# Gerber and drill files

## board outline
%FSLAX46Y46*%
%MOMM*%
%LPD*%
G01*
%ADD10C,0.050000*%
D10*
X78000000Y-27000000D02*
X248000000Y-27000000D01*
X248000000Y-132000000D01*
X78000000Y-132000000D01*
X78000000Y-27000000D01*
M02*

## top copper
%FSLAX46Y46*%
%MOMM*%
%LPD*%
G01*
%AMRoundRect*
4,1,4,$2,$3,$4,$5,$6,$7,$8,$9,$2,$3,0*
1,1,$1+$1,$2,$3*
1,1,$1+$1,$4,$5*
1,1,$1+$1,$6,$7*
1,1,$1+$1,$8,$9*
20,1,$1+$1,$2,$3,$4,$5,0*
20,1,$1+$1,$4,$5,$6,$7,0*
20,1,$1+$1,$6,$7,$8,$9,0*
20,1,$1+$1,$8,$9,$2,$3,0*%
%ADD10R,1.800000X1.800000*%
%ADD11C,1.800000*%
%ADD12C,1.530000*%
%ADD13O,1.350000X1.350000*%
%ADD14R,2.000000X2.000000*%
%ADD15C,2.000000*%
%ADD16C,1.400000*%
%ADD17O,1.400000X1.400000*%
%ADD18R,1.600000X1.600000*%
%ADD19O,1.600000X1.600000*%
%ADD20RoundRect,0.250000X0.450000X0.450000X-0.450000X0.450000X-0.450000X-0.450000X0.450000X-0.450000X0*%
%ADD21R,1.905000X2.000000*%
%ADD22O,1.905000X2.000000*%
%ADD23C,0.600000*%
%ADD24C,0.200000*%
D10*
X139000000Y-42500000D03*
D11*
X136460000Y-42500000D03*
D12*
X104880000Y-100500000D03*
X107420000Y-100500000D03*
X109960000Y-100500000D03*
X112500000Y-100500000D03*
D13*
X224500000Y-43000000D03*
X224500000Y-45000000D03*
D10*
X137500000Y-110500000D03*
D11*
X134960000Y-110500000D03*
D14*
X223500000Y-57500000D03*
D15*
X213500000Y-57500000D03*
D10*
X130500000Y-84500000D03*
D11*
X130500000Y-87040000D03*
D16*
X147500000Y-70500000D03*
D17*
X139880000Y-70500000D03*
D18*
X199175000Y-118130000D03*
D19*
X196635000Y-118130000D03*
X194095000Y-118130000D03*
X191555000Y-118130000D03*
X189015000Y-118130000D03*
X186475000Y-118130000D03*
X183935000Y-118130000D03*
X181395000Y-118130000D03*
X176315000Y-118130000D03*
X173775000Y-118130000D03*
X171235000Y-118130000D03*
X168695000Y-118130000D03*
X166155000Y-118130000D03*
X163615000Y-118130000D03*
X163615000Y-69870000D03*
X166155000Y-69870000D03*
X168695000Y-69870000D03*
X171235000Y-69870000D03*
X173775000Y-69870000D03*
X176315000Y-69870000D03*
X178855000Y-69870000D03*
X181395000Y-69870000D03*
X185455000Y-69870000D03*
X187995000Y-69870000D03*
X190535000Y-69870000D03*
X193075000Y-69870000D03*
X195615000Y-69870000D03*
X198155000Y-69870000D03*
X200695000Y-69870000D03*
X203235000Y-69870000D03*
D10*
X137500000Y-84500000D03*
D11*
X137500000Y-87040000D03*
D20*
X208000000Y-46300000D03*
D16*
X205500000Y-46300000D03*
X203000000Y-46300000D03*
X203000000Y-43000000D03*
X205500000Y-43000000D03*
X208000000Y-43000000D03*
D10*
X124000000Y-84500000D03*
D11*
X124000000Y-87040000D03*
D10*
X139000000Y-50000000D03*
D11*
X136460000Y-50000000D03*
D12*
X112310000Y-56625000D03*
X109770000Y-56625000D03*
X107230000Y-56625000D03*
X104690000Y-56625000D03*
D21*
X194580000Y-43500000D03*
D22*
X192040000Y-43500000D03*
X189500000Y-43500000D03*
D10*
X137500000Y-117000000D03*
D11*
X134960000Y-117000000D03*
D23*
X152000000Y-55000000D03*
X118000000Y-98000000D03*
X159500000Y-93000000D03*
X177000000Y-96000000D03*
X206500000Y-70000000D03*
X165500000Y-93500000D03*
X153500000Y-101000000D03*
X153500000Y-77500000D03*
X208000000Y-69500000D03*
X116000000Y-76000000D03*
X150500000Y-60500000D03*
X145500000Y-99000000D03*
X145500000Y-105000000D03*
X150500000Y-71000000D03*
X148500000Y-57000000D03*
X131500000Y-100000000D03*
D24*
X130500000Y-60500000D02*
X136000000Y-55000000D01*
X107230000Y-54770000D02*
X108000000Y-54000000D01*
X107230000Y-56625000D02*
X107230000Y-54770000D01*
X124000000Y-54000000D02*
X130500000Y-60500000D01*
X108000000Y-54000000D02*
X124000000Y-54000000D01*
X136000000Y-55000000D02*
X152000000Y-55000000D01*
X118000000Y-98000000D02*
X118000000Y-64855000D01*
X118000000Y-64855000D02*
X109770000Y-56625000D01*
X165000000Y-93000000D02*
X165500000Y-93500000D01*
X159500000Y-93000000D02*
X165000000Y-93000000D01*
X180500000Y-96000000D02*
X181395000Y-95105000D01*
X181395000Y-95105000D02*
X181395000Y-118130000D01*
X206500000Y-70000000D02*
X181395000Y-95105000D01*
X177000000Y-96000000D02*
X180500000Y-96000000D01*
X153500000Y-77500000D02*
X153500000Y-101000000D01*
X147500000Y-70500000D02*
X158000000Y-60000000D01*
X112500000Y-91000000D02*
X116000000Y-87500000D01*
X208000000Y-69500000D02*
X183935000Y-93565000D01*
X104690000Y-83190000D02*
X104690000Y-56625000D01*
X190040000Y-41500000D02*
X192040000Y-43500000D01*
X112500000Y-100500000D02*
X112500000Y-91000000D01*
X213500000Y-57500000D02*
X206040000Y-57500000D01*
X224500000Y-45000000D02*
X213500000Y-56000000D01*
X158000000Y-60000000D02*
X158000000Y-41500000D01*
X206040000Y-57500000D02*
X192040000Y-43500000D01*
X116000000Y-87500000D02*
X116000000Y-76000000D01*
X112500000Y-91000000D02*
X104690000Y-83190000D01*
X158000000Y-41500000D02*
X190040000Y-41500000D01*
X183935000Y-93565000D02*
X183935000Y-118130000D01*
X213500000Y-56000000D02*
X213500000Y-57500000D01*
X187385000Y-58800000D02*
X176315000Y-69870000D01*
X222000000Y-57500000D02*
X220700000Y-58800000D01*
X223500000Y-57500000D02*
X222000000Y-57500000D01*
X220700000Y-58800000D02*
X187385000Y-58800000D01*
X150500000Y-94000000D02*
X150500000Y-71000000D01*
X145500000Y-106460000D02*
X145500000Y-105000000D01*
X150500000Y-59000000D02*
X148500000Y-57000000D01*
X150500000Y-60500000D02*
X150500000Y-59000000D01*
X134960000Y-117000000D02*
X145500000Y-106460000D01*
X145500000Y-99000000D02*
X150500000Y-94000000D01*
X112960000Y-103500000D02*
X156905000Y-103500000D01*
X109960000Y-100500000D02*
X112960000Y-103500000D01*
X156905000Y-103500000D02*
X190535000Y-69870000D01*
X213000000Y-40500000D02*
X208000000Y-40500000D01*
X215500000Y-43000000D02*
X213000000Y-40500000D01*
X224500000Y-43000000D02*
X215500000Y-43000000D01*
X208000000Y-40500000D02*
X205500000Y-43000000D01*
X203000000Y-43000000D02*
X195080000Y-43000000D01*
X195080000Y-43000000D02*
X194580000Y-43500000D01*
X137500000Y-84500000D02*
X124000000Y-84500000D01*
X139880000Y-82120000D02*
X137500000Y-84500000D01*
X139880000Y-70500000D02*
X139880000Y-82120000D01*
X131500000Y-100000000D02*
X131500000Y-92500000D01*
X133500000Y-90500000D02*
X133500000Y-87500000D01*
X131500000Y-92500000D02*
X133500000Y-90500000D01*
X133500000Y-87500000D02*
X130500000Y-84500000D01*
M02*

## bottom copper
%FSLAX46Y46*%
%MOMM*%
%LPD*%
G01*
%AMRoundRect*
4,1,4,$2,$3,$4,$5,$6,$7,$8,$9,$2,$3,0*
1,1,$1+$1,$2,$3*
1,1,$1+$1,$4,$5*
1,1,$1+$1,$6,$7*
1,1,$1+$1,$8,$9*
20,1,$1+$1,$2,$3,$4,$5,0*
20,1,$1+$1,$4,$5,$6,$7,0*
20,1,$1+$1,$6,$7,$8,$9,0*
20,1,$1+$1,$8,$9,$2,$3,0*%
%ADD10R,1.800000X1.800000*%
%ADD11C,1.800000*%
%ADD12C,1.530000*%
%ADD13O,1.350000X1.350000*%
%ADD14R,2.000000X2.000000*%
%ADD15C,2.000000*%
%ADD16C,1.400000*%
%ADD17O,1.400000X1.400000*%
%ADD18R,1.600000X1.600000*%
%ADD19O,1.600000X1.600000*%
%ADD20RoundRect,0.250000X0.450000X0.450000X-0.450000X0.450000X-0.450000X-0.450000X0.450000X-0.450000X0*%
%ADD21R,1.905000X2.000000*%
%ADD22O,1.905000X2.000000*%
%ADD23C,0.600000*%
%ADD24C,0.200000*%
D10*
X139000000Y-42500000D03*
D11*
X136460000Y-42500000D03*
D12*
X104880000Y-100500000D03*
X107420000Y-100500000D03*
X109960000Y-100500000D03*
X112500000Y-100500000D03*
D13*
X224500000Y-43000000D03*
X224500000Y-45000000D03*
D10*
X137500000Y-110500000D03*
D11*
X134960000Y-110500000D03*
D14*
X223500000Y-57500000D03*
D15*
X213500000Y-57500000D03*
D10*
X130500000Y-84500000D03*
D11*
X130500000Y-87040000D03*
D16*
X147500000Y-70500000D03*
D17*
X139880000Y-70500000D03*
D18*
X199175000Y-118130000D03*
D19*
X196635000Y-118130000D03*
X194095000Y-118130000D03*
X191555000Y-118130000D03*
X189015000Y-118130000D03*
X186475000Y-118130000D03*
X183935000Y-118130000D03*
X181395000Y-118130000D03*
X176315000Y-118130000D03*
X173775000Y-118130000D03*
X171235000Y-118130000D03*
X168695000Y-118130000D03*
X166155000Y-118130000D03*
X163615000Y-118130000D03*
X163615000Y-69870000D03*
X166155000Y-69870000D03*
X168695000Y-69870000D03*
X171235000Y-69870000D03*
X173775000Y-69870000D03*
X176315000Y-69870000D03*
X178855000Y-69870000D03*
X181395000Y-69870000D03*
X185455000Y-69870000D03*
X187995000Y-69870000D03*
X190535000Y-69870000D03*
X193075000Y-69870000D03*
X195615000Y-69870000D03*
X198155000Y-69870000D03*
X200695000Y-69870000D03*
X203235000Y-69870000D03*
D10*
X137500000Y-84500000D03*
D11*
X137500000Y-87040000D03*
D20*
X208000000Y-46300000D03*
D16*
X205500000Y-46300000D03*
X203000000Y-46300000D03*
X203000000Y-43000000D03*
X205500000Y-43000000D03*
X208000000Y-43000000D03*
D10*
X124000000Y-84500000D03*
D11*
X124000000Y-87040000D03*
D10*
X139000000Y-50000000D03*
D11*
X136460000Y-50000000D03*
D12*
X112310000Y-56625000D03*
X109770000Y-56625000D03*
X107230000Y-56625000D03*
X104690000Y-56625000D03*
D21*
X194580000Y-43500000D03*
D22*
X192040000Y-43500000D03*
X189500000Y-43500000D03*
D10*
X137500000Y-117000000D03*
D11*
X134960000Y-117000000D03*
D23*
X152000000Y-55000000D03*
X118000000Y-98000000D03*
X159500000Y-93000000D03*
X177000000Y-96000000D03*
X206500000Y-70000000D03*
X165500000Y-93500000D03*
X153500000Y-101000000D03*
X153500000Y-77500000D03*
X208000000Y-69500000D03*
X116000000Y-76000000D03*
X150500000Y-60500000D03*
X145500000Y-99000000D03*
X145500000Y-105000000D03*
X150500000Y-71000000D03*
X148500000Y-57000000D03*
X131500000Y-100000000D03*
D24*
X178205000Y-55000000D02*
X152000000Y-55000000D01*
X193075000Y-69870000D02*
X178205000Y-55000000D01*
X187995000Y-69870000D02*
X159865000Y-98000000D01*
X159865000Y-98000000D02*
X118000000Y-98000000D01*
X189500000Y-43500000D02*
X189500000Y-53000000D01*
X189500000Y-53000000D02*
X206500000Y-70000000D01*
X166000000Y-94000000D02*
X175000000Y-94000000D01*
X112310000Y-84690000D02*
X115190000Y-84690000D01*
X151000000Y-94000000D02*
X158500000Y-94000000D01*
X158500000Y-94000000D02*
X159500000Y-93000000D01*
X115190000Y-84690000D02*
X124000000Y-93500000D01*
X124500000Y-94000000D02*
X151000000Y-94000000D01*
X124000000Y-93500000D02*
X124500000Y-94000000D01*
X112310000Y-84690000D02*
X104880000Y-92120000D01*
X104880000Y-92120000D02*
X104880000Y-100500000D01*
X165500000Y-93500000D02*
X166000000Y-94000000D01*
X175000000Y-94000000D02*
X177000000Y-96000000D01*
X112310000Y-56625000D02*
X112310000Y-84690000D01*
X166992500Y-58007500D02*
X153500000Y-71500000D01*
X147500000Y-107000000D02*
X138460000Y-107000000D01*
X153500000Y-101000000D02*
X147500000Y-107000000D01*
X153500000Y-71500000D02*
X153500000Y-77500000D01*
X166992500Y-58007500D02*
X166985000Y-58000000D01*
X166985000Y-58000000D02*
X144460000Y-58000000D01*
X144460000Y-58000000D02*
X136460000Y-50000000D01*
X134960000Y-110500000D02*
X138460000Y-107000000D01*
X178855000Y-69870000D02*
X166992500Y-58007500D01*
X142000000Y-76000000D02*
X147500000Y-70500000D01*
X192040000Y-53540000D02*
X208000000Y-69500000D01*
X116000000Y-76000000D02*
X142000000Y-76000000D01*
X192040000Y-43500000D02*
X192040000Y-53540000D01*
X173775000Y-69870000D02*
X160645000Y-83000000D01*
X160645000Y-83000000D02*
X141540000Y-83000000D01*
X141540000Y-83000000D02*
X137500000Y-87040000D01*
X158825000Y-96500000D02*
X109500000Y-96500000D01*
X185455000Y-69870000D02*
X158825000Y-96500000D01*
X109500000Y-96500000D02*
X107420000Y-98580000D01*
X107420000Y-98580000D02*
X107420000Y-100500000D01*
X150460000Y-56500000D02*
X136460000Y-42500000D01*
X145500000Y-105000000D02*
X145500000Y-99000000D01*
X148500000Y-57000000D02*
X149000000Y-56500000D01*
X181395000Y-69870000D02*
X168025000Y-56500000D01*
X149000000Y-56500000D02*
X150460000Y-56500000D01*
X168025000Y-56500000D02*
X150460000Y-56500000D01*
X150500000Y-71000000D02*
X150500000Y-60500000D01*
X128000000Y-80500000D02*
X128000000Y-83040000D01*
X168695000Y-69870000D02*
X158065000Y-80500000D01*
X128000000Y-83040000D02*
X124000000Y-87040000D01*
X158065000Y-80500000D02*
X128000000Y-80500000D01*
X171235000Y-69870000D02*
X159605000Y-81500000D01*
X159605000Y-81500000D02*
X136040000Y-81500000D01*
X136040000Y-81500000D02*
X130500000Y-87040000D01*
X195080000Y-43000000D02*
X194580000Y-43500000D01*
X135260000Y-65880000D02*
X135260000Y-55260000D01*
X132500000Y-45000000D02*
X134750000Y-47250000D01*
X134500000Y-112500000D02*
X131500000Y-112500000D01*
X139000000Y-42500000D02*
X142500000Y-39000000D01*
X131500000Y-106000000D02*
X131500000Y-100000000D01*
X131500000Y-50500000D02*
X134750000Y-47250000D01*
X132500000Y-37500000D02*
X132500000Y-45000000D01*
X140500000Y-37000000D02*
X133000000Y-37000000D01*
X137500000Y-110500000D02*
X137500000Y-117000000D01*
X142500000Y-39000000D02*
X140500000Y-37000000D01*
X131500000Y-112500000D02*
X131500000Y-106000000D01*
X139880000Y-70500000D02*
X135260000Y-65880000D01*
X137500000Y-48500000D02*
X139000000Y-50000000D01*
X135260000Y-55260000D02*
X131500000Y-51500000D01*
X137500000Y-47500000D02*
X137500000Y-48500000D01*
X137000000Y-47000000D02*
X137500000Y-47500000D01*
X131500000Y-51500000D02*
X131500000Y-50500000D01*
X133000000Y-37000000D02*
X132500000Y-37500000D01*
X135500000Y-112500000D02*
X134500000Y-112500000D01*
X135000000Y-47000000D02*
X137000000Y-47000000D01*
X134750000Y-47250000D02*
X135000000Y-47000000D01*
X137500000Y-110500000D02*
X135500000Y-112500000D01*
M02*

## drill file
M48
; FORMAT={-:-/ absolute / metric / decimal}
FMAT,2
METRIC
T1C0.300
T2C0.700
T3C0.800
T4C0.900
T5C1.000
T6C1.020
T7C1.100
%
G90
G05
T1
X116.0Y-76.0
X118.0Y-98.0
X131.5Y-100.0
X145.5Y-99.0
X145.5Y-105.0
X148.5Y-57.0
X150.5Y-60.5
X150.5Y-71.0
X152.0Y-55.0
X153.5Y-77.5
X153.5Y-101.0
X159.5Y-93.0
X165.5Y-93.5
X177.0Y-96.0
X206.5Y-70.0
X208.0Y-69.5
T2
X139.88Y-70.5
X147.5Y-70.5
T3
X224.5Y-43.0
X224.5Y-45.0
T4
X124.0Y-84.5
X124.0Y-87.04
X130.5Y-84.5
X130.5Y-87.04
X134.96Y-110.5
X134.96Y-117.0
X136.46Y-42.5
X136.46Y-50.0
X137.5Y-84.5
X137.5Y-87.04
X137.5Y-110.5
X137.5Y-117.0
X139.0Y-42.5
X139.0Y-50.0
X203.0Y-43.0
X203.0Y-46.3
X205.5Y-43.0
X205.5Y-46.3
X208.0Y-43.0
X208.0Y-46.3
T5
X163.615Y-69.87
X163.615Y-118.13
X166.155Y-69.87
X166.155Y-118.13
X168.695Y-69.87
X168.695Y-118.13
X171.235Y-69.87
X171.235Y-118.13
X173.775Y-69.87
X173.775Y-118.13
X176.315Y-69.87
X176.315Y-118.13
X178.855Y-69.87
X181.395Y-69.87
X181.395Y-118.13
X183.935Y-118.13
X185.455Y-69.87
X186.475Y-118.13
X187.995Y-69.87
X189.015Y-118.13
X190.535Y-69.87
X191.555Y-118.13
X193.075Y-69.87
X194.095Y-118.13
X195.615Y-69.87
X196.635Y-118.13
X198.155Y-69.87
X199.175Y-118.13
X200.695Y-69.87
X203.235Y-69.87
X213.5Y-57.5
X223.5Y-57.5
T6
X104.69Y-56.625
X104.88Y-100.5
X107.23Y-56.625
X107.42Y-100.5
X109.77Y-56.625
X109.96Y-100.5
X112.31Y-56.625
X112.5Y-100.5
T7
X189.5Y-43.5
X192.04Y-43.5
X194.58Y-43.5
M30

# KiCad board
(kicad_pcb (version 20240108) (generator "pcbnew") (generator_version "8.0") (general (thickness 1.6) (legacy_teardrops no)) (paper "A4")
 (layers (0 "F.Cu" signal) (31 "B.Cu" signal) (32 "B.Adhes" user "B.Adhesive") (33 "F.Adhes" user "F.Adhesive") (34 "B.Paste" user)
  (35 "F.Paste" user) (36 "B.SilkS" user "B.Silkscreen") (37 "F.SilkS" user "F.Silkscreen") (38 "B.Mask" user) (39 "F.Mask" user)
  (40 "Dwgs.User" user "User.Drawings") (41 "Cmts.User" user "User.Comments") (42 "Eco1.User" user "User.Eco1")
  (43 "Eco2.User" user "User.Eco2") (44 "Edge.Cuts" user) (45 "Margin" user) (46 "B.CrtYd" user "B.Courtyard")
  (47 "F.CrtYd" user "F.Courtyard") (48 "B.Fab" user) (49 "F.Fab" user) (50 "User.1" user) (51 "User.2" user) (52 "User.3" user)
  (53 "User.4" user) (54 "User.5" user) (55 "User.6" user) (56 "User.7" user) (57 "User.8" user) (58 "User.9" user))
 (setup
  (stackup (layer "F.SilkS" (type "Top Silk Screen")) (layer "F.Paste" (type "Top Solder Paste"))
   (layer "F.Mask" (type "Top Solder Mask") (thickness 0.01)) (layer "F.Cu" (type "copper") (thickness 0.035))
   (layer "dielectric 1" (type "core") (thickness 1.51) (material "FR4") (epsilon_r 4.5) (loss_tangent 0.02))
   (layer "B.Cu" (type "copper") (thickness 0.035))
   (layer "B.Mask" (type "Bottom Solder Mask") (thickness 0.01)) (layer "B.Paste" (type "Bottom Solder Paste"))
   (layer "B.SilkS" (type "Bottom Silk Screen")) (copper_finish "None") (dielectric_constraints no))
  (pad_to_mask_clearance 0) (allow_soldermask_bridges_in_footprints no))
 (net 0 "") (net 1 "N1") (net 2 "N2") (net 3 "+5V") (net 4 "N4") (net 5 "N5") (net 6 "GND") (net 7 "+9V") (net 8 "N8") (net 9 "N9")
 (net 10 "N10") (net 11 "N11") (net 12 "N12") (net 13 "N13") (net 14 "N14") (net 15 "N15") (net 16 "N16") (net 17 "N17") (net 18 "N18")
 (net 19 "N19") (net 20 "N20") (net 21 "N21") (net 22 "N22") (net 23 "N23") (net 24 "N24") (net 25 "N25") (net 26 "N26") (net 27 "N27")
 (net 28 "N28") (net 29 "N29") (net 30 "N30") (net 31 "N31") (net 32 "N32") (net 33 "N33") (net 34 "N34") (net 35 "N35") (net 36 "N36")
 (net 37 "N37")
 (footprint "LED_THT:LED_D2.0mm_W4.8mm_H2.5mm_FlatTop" (layer "F.Cu") (at 139 42.5 180)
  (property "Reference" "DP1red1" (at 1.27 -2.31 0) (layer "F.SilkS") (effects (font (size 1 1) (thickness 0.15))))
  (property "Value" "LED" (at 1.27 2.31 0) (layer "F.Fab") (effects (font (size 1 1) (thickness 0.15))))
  (pad "1" thru_hole rect (at 0 0 180) (size 1.8 1.8) (drill 0.9) (layers "*.Cu" "*.Mask") (remove_unused_layers no) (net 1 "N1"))
  (pad "2" thru_hole circle (at 2.54 0 180) (size 1.8 1.8) (drill 0.9) (layers "*.Cu" "*.Mask") (remove_unused_layers no) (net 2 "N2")))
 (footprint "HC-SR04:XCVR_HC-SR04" (layer "F.Cu") (at 108.69 100.5)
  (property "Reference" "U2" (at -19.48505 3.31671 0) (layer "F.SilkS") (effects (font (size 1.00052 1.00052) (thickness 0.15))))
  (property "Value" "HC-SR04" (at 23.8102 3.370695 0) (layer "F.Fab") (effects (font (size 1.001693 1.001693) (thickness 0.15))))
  (pad "1" thru_hole circle (at -3.81 0) (size 1.53 1.53) (drill 1.02) (layers "*.Cu" "*.Mask") (remove_unused_layers no) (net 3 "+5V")
   (solder_mask_margin 0.102))
  (pad "2" thru_hole circle (at -1.27 0) (size 1.53 1.53) (drill 1.02) (layers "*.Cu" "*.Mask") (remove_unused_layers no) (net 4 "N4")
   (solder_mask_margin 0.102))
  (pad "3" thru_hole circle (at 1.27 0) (size 1.53 1.53) (drill 1.02) (layers "*.Cu" "*.Mask") (remove_unused_layers no) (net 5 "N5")
   (solder_mask_margin 0.102))
  (pad "4" thru_hole circle (at 3.81 0) (size 1.53 1.53) (drill 1.02) (layers "*.Cu" "*.Mask") (remove_unused_layers no) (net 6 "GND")
   (solder_mask_margin 0.102)))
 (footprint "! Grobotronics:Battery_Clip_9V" (layer "F.Cu") (at 224.5 43.5)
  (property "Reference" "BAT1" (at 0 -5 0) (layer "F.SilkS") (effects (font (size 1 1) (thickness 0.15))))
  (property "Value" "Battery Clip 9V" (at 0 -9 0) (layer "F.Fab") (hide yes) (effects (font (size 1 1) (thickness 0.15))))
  (pad "+" thru_hole oval (at 0 -0.5) (size 1.35 1.35) (drill 0.8) (layers "*.Cu" "*.Mask") (remove_unused_layers no) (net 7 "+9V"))
  (pad "-" thru_hole oval (at 0 1.5) (size 1.35 1.35) (drill 0.8) (layers "*.Cu" "*.Mask") (remove_unused_layers no) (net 6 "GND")))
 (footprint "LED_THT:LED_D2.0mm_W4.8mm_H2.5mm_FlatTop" (layer "F.Cu") (at 137.5 110.5 180)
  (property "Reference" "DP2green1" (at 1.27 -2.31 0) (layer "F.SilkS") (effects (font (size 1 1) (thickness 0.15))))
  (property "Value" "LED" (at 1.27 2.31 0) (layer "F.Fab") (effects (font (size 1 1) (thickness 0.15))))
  (pad "1" thru_hole rect (at 0 0 180) (size 1.8 1.8) (drill 0.9) (layers "*.Cu" "*.Mask") (remove_unused_layers no) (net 1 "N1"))
  (pad "2" thru_hole circle (at 2.54 0 180) (size 1.8 1.8) (drill 0.9) (layers "*.Cu" "*.Mask") (remove_unused_layers no) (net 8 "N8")))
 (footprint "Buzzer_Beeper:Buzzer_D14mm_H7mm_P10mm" (layer "F.Cu") (at 223.5 57.5 180)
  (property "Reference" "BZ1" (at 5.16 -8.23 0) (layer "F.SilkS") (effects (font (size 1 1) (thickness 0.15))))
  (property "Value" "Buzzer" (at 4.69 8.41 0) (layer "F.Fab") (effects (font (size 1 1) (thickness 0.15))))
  (pad "1" thru_hole rect (at 0 0 180) (size 2 2) (drill 1) (layers "*.Cu" "*.Mask") (remove_unused_layers no) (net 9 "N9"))
  (pad "2" thru_hole circle (at 10 0 180) (size 2 2) (drill 1) (layers "*.Cu" "*.Mask") (remove_unused_layers no) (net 6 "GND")))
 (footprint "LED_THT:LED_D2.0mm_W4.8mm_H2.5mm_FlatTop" (layer "F.Cu") (at 130.5 84.5 -90)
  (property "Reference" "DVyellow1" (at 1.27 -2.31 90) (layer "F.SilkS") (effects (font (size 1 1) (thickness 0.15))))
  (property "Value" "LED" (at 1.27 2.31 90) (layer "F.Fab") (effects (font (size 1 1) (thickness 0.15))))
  (pad "1" thru_hole rect (at 0 0 270) (size 1.8 1.8) (drill 0.9) (layers "*.Cu" "*.Mask") (remove_unused_layers no) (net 1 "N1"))
  (pad "2" thru_hole circle (at 2.54 0 270) (size 1.8 1.8) (drill 0.9) (layers "*.Cu" "*.Mask") (remove_unused_layers no) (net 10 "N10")))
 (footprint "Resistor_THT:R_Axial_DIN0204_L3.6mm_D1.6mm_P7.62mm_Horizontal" (layer "F.Cu") (at 147.5 70.5 180)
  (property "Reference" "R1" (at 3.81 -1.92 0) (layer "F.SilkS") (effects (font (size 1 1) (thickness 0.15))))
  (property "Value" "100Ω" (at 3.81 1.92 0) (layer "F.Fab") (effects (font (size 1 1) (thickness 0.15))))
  (pad "1" thru_hole circle (at 0 0 180) (size 1.4 1.4) (drill 0.7) (layers "*.Cu" "*.Mask") (remove_unused_layers no) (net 6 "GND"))
  (pad "2" thru_hole oval (at 7.62 0 180) (size 1.4 1.4) (drill 0.7) (layers "*.Cu" "*.Mask") (remove_unused_layers no) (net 1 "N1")))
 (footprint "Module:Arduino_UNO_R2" (layer "F.Cu") (at 199.175 118.13 180)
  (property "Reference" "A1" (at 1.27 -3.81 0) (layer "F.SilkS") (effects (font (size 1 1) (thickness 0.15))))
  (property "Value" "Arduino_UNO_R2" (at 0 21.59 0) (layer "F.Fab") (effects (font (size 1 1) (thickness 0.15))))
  (pad "1" thru_hole rect (at 0 0 270) (size 1.6 1.6) (drill 1) (layers "*.Cu" "*.Mask") (remove_unused_layers no) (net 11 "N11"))
  (pad "2" thru_hole oval (at 2.54 0 270) (size 1.6 1.6) (drill 1) (layers "*.Cu" "*.Mask") (remove_unused_layers no) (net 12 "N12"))
  (pad "3" thru_hole oval (at 5.08 0 270) (size 1.6 1.6) (drill 1) (layers "*.Cu" "*.Mask") (remove_unused_layers no) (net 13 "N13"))
  (pad "4" thru_hole oval (at 7.62 0 270) (size 1.6 1.6) (drill 1) (layers "*.Cu" "*.Mask") (remove_unused_layers no) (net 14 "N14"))
  (pad "5" thru_hole oval (at 10.16 0 270) (size 1.6 1.6) (drill 1) (layers "*.Cu" "*.Mask") (remove_unused_layers no) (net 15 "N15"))
  (pad "6" thru_hole oval (at 12.7 0 270) (size 1.6 1.6) (drill 1) (layers "*.Cu" "*.Mask") (remove_unused_layers no) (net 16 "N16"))
  (pad "7" thru_hole oval (at 15.24 0 270) (size 1.6 1.6) (drill 1) (layers "*.Cu" "*.Mask") (remove_unused_layers no) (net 6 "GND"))
  (pad "8" thru_hole oval (at 17.78 0 270) (size 1.6 1.6) (drill 1) (layers "*.Cu" "*.Mask") (remove_unused_layers no) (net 3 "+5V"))
  (pad "9" thru_hole oval (at 22.86 0 270) (size 1.6 1.6) (drill 1) (layers "*.Cu" "*.Mask") (remove_unused_layers no) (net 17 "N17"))
  (pad "10" thru_hole oval (at 25.4 0 270) (size 1.6 1.6) (drill 1) (layers "*.Cu" "*.Mask") (remove_unused_layers no) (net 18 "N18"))
  (pad "11" thru_hole oval (at 27.94 0 270) (size 1.6 1.6) (drill 1) (layers "*.Cu" "*.Mask") (remove_unused_layers no) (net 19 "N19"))
  (pad "12" thru_hole oval (at 30.48 0 270) (size 1.6 1.6) (drill 1) (layers "*.Cu" "*.Mask") (remove_unused_layers no) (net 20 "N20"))
  (pad "13" thru_hole oval (at 33.02 0 270) (size 1.6 1.6) (drill 1) (layers "*.Cu" "*.Mask") (remove_unused_layers no) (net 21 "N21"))
  (pad "14" thru_hole oval (at 35.56 0 270) (size 1.6 1.6) (drill 1) (layers "*.Cu" "*.Mask") (remove_unused_layers no) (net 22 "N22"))
  (pad "15" thru_hole oval (at 35.56 48.26 270) (size 1.6 1.6) (drill 1) (layers "*.Cu" "*.Mask") (remove_unused_layers no) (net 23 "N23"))
  (pad "16" thru_hole oval (at 33.02 48.26 270) (size 1.6 1.6) (drill 1) (layers "*.Cu" "*.Mask") (remove_unused_layers no) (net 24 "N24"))
  (pad "17" thru_hole oval (at 30.48 48.26 270) (size 1.6 1.6) (drill 1) (layers "*.Cu" "*.Mask") (remove_unused_layers no) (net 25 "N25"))
  (pad "18" thru_hole oval (at 27.94 48.26 270) (size 1.6 1.6) (drill 1) (layers "*.Cu" "*.Mask") (remove_unused_layers no) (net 10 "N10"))
  (pad "19" thru_hole oval (at 25.4 48.26 270) (size 1.6 1.6) (drill 1) (layers "*.Cu" "*.Mask") (remove_unused_layers no) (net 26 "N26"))
  (pad "20" thru_hole oval (at 22.86 48.26 270) (size 1.6 1.6) (drill 1) (layers "*.Cu" "*.Mask") (remove_unused_layers no) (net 9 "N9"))
  (pad "21" thru_hole oval (at 20.32 48.26 270) (size 1.6 1.6) (drill 1) (layers "*.Cu" "*.Mask") (remove_unused_layers no) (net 8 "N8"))
  (pad "22" thru_hole oval (at 17.78 48.26 270) (size 1.6 1.6) (drill 1) (layers "*.Cu" "*.Mask") (remove_unused_layers no) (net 2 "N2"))
  (pad "23" thru_hole oval (at 13.72 48.26 270) (size 1.6 1.6) (drill 1) (layers "*.Cu" "*.Mask") (remove_unused_layers no) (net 4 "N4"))
  (pad "24" thru_hole oval (at 11.18 48.26 270) (size 1.6 1.6) (drill 1) (layers "*.Cu" "*.Mask") (remove_unused_layers no) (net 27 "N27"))
  (pad "25" thru_hole oval (at 8.64 48.26 270) (size 1.6 1.6) (drill 1) (layers "*.Cu" "*.Mask") (remove_unused_layers no) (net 5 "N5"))
  (pad "26" thru_hole oval (at 6.1 48.26 270) (size 1.6 1.6) (drill 1) (layers "*.Cu" "*.Mask") (remove_unused_layers no) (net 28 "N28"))
  (pad "27" thru_hole oval (at 3.56 48.26 270) (size 1.6 1.6) (drill 1) (layers "*.Cu" "*.Mask") (remove_unused_layers no) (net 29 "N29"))
  (pad "28" thru_hole oval (at 1.02 48.26 270) (size 1.6 1.6) (drill 1) (layers "*.Cu" "*.Mask") (remove_unused_layers no) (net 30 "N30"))
  (pad "29" thru_hole oval (at -1.52 48.26 270) (size 1.6 1.6) (drill 1) (layers "*.Cu" "*.Mask") (remove_unused_layers no) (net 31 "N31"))
  (pad "30" thru_hole oval (at -4.06 48.26 270) (size 1.6 1.6) (drill 1) (layers "*.Cu" "*.Mask") (remove_unused_layers no) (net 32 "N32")))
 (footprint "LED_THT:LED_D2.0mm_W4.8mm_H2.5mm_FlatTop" (layer "F.Cu") (at 137.5 84.5 -90)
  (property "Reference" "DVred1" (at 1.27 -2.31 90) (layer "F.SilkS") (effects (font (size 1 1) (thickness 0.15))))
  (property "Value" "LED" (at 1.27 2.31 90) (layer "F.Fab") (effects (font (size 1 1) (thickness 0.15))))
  (pad "1" thru_hole rect (at 0 0 270) (size 1.8 1.8) (drill 0.9) (layers "*.Cu" "*.Mask") (remove_unused_layers no) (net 1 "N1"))
  (pad "2" thru_hole circle (at 2.54 0 270) (size 1.8 1.8) (drill 0.9) (layers "*.Cu" "*.Mask") (remove_unused_layers no) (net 26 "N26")))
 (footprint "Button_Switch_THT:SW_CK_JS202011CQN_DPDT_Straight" (layer "F.Cu") (at 208 46.3 180)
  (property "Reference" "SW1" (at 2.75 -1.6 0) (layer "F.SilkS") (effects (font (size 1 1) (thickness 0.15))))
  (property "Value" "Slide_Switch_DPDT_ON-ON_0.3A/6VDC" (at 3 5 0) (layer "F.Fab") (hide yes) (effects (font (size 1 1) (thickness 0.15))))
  (pad "1" thru_hole roundrect (at 0 0 180) (size 1.4 1.4) (drill 0.9) (layers "*.Cu" "*.Mask") (remove_unused_layers no)
   (roundrect_rratio 0.1785714286) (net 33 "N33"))
  (pad "2" thru_hole circle (at 2.5 0 180) (size 1.4 1.4) (drill 0.9) (layers "*.Cu" "*.Mask") (remove_unused_layers no) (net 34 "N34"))
  (pad "3" thru_hole circle (at 5 0 180) (size 1.4 1.4) (drill 0.9) (layers "*.Cu" "*.Mask") (remove_unused_layers no) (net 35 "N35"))
  (pad "4" thru_hole circle (at 5 3.3 180) (size 1.4 1.4) (drill 0.9) (layers "*.Cu" "*.Mask") (remove_unused_layers no) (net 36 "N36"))
  (pad "5" thru_hole circle (at 2.5 3.3 180) (size 1.4 1.4) (drill 0.9) (layers "*.Cu" "*.Mask") (remove_unused_layers no) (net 7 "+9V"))
  (pad "6" thru_hole circle (at 0 3.3 180) (size 1.4 1.4) (drill 0.9) (layers "*.Cu" "*.Mask") (remove_unused_layers no) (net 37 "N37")))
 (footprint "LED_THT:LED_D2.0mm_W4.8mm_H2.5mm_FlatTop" (layer "F.Cu") (at 124 84.5 -90)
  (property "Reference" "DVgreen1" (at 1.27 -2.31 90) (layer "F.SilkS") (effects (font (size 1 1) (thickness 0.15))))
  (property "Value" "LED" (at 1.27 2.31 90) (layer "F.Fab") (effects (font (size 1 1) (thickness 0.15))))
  (pad "1" thru_hole rect (at 0 0 270) (size 1.8 1.8) (drill 0.9) (layers "*.Cu" "*.Mask") (remove_unused_layers no) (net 1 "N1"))
  (pad "2" thru_hole circle (at 2.54 0 270) (size 1.8 1.8) (drill 0.9) (layers "*.Cu" "*.Mask") (remove_unused_layers no) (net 25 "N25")))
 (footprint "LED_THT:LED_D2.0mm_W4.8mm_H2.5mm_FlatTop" (layer "F.Cu") (at 139 50 180)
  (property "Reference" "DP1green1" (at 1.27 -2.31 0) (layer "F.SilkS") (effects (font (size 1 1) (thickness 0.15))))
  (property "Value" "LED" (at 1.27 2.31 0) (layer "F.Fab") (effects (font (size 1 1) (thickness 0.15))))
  (pad "1" thru_hole rect (at 0 0 180) (size 1.8 1.8) (drill 0.9) (layers "*.Cu" "*.Mask") (remove_unused_layers no) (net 1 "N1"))
  (pad "2" thru_hole circle (at 2.54 0 180) (size 1.8 1.8) (drill 0.9) (layers "*.Cu" "*.Mask") (remove_unused_layers no) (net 8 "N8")))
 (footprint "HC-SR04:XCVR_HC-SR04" (layer "F.Cu") (at 108.5 56.625 180)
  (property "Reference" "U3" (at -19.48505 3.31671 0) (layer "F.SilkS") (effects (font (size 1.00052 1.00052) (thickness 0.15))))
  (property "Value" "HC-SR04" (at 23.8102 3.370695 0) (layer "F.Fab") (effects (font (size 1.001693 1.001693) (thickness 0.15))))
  (pad "1" thru_hole circle (at -3.81 0 180) (size 1.53 1.53) (drill 1.02) (layers "*.Cu" "*.Mask") (remove_unused_layers no) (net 3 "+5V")
   (solder_mask_margin 0.102))
  (pad "2" thru_hole circle (at -1.27 0 180) (size 1.53 1.53) (drill 1.02) (layers "*.Cu" "*.Mask") (remove_unused_layers no) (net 27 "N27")
   (solder_mask_margin 0.102))
  (pad "3" thru_hole circle (at 1.27 0 180) (size 1.53 1.53) (drill 1.02) (layers "*.Cu" "*.Mask") (remove_unused_layers no) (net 28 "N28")
   (solder_mask_margin 0.102))
  (pad "4" thru_hole circle (at 3.81 0 180) (size 1.53 1.53) (drill 1.02) (layers "*.Cu" "*.Mask") (remove_unused_layers no) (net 6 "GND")
   (solder_mask_margin 0.102)))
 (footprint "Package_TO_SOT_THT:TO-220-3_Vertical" (layer "F.Cu") (at 194.58 43.5 180)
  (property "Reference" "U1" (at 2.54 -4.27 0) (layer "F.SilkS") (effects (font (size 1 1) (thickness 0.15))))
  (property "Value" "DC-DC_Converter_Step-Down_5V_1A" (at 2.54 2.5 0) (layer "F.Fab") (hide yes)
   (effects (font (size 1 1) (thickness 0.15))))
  (pad "1" thru_hole rect (at 0 0 180) (size 1.905 2) (drill 1.1) (layers "*.Cu" "*.Mask") (remove_unused_layers no) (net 36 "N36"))
  (pad "2" thru_hole oval (at 2.54 0 180) (size 1.905 2) (drill 1.1) (layers "*.Cu" "*.Mask") (remove_unused_layers no) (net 6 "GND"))
  (pad "3" thru_hole oval (at 5.08 0 180) (size 1.905 2) (drill 1.1) (layers "*.Cu" "*.Mask") (remove_unused_layers no) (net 3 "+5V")))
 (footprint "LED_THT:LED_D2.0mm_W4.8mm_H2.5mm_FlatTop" (layer "F.Cu") (at 137.5 117 180)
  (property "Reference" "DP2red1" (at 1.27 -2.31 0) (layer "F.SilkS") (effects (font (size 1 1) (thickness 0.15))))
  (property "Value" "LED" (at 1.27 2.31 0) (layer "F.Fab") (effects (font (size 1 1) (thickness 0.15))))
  (pad "1" thru_hole rect (at 0 0 180) (size 1.8 1.8) (drill 0.9) (layers "*.Cu" "*.Mask") (remove_unused_layers no) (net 1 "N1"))
  (pad "2" thru_hole circle (at 2.54 0 180) (size 1.8 1.8) (drill 0.9) (layers "*.Cu" "*.Mask") (remove_unused_layers no) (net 2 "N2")))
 (gr_rect (start 78 27) (end 248 132) (stroke (width 0.05) (type default)) (fill none) (layer "Edge.Cuts"))
 (segment (start 130.5 60.5) (end 136 55) (width 0.2) (layer "F.Cu") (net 28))
 (segment (start 107.23 54.77) (end 108 54) (width 0.2) (layer "F.Cu") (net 28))
 (segment (start 107.23 56.625) (end 107.23 54.77) (width 0.2) (layer "F.Cu") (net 28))
 (segment (start 124 54) (end 130.5 60.5) (width 0.2) (layer "F.Cu") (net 28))
 (segment (start 108 54) (end 124 54) (width 0.2) (layer "F.Cu") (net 28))
 (segment (start 136 55) (end 152 55) (width 0.2) (layer "F.Cu") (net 28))
 (via (at 152 55) (size 0.6) (drill 0.3) (layers "F.Cu" "B.Cu") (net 28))
 (segment (start 178.205 55) (end 152 55) (width 0.2) (layer "B.Cu") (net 28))
 (segment (start 193.075 69.87) (end 178.205 55) (width 0.2) (layer "B.Cu") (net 28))
 (segment (start 118 98) (end 118 64.855) (width 0.2) (layer "F.Cu") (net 27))
 (segment (start 118 64.855) (end 109.77 56.625) (width 0.2) (layer "F.Cu") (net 27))
 (via (at 118 98) (size 0.6) (drill 0.3) (layers "F.Cu" "B.Cu") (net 27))
 (segment (start 187.995 69.87) (end 159.865 98) (width 0.2) (layer "B.Cu") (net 27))
 (segment (start 159.865 98) (end 118 98) (width 0.2) (layer "B.Cu") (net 27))
 (segment (start 165 93) (end 165.5 93.5) (width 0.2) (layer "F.Cu") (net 3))
 (segment (start 159.5 93) (end 165 93) (width 0.2) (layer "F.Cu") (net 3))
 (segment (start 180.5 96) (end 181.395 95.105) (width 0.2) (layer "F.Cu") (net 3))
 (segment (start 181.395 95.105) (end 181.395 118.13) (width 0.2) (layer "F.Cu") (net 3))
 (segment (start 206.5 70) (end 181.395 95.105) (width 0.2) (layer "F.Cu") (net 3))
 (segment (start 177 96) (end 180.5 96) (width 0.2) (layer "F.Cu") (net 3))
 (via (at 159.5 93) (size 0.6) (drill 0.3) (layers "F.Cu" "B.Cu") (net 3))
 (via (at 177 96) (size 0.6) (drill 0.3) (layers "F.Cu" "B.Cu") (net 3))
 (via (at 206.5 70) (size 0.6) (drill 0.3) (layers "F.Cu" "B.Cu") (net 3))
 (via (at 165.5 93.5) (size 0.6) (drill 0.3) (layers "F.Cu" "B.Cu") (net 3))
 (segment (start 189.5 43.5) (end 189.5 53) (width 0.2) (layer "B.Cu") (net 3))
 (segment (start 189.5 53) (end 206.5 70) (width 0.2) (layer "B.Cu") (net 3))
 (segment (start 166 94) (end 175 94) (width 0.2) (layer "B.Cu") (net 3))
 (segment (start 112.31 84.69) (end 115.19 84.69) (width 0.2) (layer "B.Cu") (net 3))
 (segment (start 151 94) (end 158.5 94) (width 0.2) (layer "B.Cu") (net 3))
 (segment (start 158.5 94) (end 159.5 93) (width 0.2) (layer "B.Cu") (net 3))
 (segment (start 115.19 84.69) (end 124 93.5) (width 0.2) (layer "B.Cu") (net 3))
 (segment (start 124.5 94) (end 151 94) (width 0.2) (layer "B.Cu") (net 3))
 (segment (start 124 93.5) (end 124.5 94) (width 0.2) (layer "B.Cu") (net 3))
 (segment (start 112.31 84.69) (end 104.88 92.12) (width 0.2) (layer "B.Cu") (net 3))
 (segment (start 104.88 92.12) (end 104.88 100.5) (width 0.2) (layer "B.Cu") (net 3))
 (segment (start 165.5 93.5) (end 166 94) (width 0.2) (layer "B.Cu") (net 3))
 (segment (start 175 94) (end 177 96) (width 0.2) (layer "B.Cu") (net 3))
 (segment (start 112.31 56.625) (end 112.31 84.69) (width 0.2) (layer "B.Cu") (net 3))
 (segment (start 153.5 77.5) (end 153.5 101) (width 0.2) (layer "F.Cu") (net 8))
 (via (at 153.5 101) (size 0.6) (drill 0.3) (layers "F.Cu" "B.Cu") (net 8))
 (via (at 153.5 77.5) (size 0.6) (drill 0.3) (layers "F.Cu" "B.Cu") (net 8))
 (segment (start 166.9925 58.0075) (end 153.5 71.5) (width 0.2) (layer "B.Cu") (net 8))
 (segment (start 147.5 107) (end 138.46 107) (width 0.2) (layer "B.Cu") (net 8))
 (segment (start 153.5 101) (end 147.5 107) (width 0.2) (layer "B.Cu") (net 8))
 (segment (start 153.5 71.5) (end 153.5 77.5) (width 0.2) (layer "B.Cu") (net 8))
 (segment (start 166.9925 58.0075) (end 166.985 58) (width 0.2) (layer "B.Cu") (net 8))
 (segment (start 166.985 58) (end 144.46 58) (width 0.2) (layer "B.Cu") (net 8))
 (segment (start 144.46 58) (end 136.46 50) (width 0.2) (layer "B.Cu") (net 8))
 (segment (start 134.96 110.5) (end 138.46 107) (width 0.2) (layer "B.Cu") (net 8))
 (segment (start 178.855 69.87) (end 166.9925 58.0075) (width 0.2) (layer "B.Cu") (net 8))
 (segment (start 147.5 70.5) (end 158 60) (width 0.2) (layer "F.Cu") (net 6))
 (segment (start 112.5 91) (end 116 87.5) (width 0.2) (layer "F.Cu") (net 6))
 (segment (start 208 69.5) (end 183.935 93.565) (width 0.2) (layer "F.Cu") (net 6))
 (segment (start 104.69 83.19) (end 104.69 56.625) (width 0.2) (layer "F.Cu") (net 6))
 (segment (start 190.04 41.5) (end 192.04 43.5) (width 0.2) (layer "F.Cu") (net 6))
 (segment (start 112.5 100.5) (end 112.5 91) (width 0.2) (layer "F.Cu") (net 6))
 (segment (start 213.5 57.5) (end 206.04 57.5) (width 0.2) (layer "F.Cu") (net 6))
 (segment (start 224.5 45) (end 213.5 56) (width 0.2) (layer "F.Cu") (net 6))
 (segment (start 158 60) (end 158 41.5) (width 0.2) (layer "F.Cu") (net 6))
 (segment (start 206.04 57.5) (end 192.04 43.5) (width 0.2) (layer "F.Cu") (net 6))
 (segment (start 116 87.5) (end 116 76) (width 0.2) (layer "F.Cu") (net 6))
 (segment (start 112.5 91) (end 104.69 83.19) (width 0.2) (layer "F.Cu") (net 6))
 (segment (start 158 41.5) (end 190.04 41.5) (width 0.2) (layer "F.Cu") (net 6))
 (segment (start 183.935 93.565) (end 183.935 118.13) (width 0.2) (layer "F.Cu") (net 6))
 (segment (start 213.5 56) (end 213.5 57.5) (width 0.2) (layer "F.Cu") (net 6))
 (via (at 208 69.5) (size 0.6) (drill 0.3) (layers "F.Cu" "B.Cu") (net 6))
 (via (at 116 76) (size 0.6) (drill 0.3) (layers "F.Cu" "B.Cu") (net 6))
 (segment (start 142 76) (end 147.5 70.5) (width 0.2) (layer "B.Cu") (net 6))
 (segment (start 192.04 53.54) (end 208 69.5) (width 0.2) (layer "B.Cu") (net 6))
 (segment (start 116 76) (end 142 76) (width 0.2) (layer "B.Cu") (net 6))
 (segment (start 192.04 43.5) (end 192.04 53.54) (width 0.2) (layer "B.Cu") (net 6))
 (segment (start 173.775 69.87) (end 160.645 83) (width 0.2) (layer "B.Cu") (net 26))
 (segment (start 160.645 83) (end 141.54 83) (width 0.2) (layer "B.Cu") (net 26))
 (segment (start 141.54 83) (end 137.5 87.04) (width 0.2) (layer "B.Cu") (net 26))
 (segment (start 187.385 58.8) (end 176.315 69.87) (width 0.2) (layer "F.Cu") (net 9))
 (segment (start 222 57.5) (end 220.7 58.8) (width 0.2) (layer "F.Cu") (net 9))
 (segment (start 223.5 57.5) (end 222 57.5) (width 0.2) (layer "F.Cu") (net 9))
 (segment (start 220.7 58.8) (end 187.385 58.8) (width 0.2) (layer "F.Cu") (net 9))
 (segment (start 158.825 96.5) (end 109.5 96.5) (width 0.2) (layer "B.Cu") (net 4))
 (segment (start 185.455 69.87) (end 158.825 96.5) (width 0.2) (layer "B.Cu") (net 4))
 (segment (start 109.5 96.5) (end 107.42 98.58) (width 0.2) (layer "B.Cu") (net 4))
 (segment (start 107.42 98.58) (end 107.42 100.5) (width 0.2) (layer "B.Cu") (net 4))
 (segment (start 150.5 94) (end 150.5 71) (width 0.2) (layer "F.Cu") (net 2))
 (segment (start 145.5 106.46) (end 145.5 105) (width 0.2) (layer "F.Cu") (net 2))
 (segment (start 150.5 59) (end 148.5 57) (width 0.2) (layer "F.Cu") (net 2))
 (segment (start 150.5 60.5) (end 150.5 59) (width 0.2) (layer "F.Cu") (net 2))
 (segment (start 134.96 117) (end 145.5 106.46) (width 0.2) (layer "F.Cu") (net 2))
 (segment (start 145.5 99) (end 150.5 94) (width 0.2) (layer "F.Cu") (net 2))
 (via (at 150.5 60.5) (size 0.6) (drill 0.3) (layers "F.Cu" "B.Cu") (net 2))
 (via (at 145.5 99) (size 0.6) (drill 0.3) (layers "F.Cu" "B.Cu") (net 2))
 (via (at 145.5 105) (size 0.6) (drill 0.3) (layers "F.Cu" "B.Cu") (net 2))
 (via (at 150.5 71) (size 0.6) (drill 0.3) (layers "F.Cu" "B.Cu") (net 2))
 (via (at 148.5 57) (size 0.6) (drill 0.3) (layers "F.Cu" "B.Cu") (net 2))
 (segment (start 150.46 56.5) (end 136.46 42.5) (width 0.2) (layer "B.Cu") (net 2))
 (segment (start 145.5 105) (end 145.5 99) (width 0.2) (layer "B.Cu") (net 2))
 (segment (start 148.5 57) (end 149 56.5) (width 0.2) (layer "B.Cu") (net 2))
 (segment (start 181.395 69.87) (end 168.025 56.5) (width 0.2) (layer "B.Cu") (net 2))
 (segment (start 149 56.5) (end 150.46 56.5) (width 0.2) (layer "B.Cu") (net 2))
 (segment (start 168.025 56.5) (end 150.46 56.5) (width 0.2) (layer "B.Cu") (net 2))
 (segment (start 150.5 71) (end 150.5 60.5) (width 0.2) (layer "B.Cu") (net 2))
 (segment (start 128 80.5) (end 128 83.04) (width 0.2) (layer "B.Cu") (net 25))
 (segment (start 168.695 69.87) (end 158.065 80.5) (width 0.2) (layer "B.Cu") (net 25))
 (segment (start 128 83.04) (end 124 87.04) (width 0.2) (layer "B.Cu") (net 25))
 (segment (start 158.065 80.5) (end 128 80.5) (width 0.2) (layer "B.Cu") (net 25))
 (segment (start 171.235 69.87) (end 159.605 81.5) (width 0.2) (layer "B.Cu") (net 10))
 (segment (start 159.605 81.5) (end 136.04 81.5) (width 0.2) (layer "B.Cu") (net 10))
 (segment (start 136.04 81.5) (end 130.5 87.04) (width 0.2) (layer "B.Cu") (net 10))
 (segment (start 112.96 103.5) (end 156.905 103.5) (width 0.2) (layer "F.Cu") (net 5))
 (segment (start 109.96 100.5) (end 112.96 103.5) (width 0.2) (layer "F.Cu") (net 5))
 (segment (start 156.905 103.5) (end 190.535 69.87) (width 0.2) (layer "F.Cu") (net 5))
 (segment (start 213 40.5) (end 208 40.5) (width 0.2) (layer "F.Cu") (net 7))
 (segment (start 215.5 43) (end 213 40.5) (width 0.2) (layer "F.Cu") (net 7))
 (segment (start 224.5 43) (end 215.5 43) (width 0.2) (layer "F.Cu") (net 7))
 (segment (start 208 40.5) (end 205.5 43) (width 0.2) (layer "F.Cu") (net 7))
 (segment (start 203 43) (end 195.08 43) (width 0.2) (layer "F.Cu") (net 36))
 (segment (start 195.08 43) (end 194.58 43.5) (width 0.2) (layer "F.Cu") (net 36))
 (segment (start 195.08 43) (end 194.58 43.5) (width 0.2) (layer "B.Cu") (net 36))
 (segment (start 137.5 84.5) (end 124 84.5) (width 0.2) (layer "F.Cu") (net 1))
 (segment (start 139.88 82.12) (end 137.5 84.5) (width 0.2) (layer "F.Cu") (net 1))
 (segment (start 139.88 70.5) (end 139.88 82.12) (width 0.2) (layer "F.Cu") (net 1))
 (segment (start 131.5 100) (end 131.5 92.5) (width 0.2) (layer "F.Cu") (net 1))
 (segment (start 133.5 90.5) (end 133.5 87.5) (width 0.2) (layer "F.Cu") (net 1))
 (segment (start 131.5 92.5) (end 133.5 90.5) (width 0.2) (layer "F.Cu") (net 1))
 (segment (start 133.5 87.5) (end 130.5 84.5) (width 0.2) (layer "F.Cu") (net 1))
 (via (at 131.5 100) (size 0.6) (drill 0.3) (layers "F.Cu" "B.Cu") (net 1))
 (segment (start 135.26 65.88) (end 135.26 55.26) (width 0.2) (layer "B.Cu") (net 1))
 (segment (start 132.5 45) (end 134.75 47.25) (width 0.2) (layer "B.Cu") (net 1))
 (segment (start 134.5 112.5) (end 131.5 112.5) (width 0.2) (layer "B.Cu") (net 1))
 (segment (start 139 42.5) (end 142.5 39) (width 0.2) (layer "B.Cu") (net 1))
 (segment (start 131.5 106) (end 131.5 100) (width 0.2) (layer "B.Cu") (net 1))
 (segment (start 131.5 50.5) (end 134.75 47.25) (width 0.2) (layer "B.Cu") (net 1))
 (segment (start 132.5 37.5) (end 132.5 45) (width 0.2) (layer "B.Cu") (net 1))
 (segment (start 140.5 37) (end 133 37) (width 0.2) (layer "B.Cu") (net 1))
 (segment (start 137.5 110.5) (end 137.5 117) (width 0.2) (layer "B.Cu") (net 1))
 (segment (start 142.5 39) (end 140.5 37) (width 0.2) (layer "B.Cu") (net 1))
 (segment (start 131.5 112.5) (end 131.5 106) (width 0.2) (layer "B.Cu") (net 1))
 (segment (start 139.88 70.5) (end 135.26 65.88) (width 0.2) (layer "B.Cu") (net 1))
 (segment (start 137.5 48.5) (end 139 50) (width 0.2) (layer "B.Cu") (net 1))
 (segment (start 135.26 55.26) (end 131.5 51.5) (width 0.2) (layer "B.Cu") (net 1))
 (segment (start 137.5 47.5) (end 137.5 48.5) (width 0.2) (layer "B.Cu") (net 1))
 (segment (start 137 47) (end 137.5 47.5) (width 0.2) (layer "B.Cu") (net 1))
 (segment (start 131.5 51.5) (end 131.5 50.5) (width 0.2) (layer "B.Cu") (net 1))
 (segment (start 133 37) (end 132.5 37.5) (width 0.2) (layer "B.Cu") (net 1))
 (segment (start 135.5 112.5) (end 134.5 112.5) (width 0.2) (layer "B.Cu") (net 1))
 (segment (start 135 47) (end 137 47) (width 0.2) (layer "B.Cu") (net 1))
 (segment (start 134.75 47.25) (end 135 47) (width 0.2) (layer "B.Cu") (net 1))
 (segment (start 137.5 110.5) (end 135.5 112.5) (width 0.2) (layer "B.Cu") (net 1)))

